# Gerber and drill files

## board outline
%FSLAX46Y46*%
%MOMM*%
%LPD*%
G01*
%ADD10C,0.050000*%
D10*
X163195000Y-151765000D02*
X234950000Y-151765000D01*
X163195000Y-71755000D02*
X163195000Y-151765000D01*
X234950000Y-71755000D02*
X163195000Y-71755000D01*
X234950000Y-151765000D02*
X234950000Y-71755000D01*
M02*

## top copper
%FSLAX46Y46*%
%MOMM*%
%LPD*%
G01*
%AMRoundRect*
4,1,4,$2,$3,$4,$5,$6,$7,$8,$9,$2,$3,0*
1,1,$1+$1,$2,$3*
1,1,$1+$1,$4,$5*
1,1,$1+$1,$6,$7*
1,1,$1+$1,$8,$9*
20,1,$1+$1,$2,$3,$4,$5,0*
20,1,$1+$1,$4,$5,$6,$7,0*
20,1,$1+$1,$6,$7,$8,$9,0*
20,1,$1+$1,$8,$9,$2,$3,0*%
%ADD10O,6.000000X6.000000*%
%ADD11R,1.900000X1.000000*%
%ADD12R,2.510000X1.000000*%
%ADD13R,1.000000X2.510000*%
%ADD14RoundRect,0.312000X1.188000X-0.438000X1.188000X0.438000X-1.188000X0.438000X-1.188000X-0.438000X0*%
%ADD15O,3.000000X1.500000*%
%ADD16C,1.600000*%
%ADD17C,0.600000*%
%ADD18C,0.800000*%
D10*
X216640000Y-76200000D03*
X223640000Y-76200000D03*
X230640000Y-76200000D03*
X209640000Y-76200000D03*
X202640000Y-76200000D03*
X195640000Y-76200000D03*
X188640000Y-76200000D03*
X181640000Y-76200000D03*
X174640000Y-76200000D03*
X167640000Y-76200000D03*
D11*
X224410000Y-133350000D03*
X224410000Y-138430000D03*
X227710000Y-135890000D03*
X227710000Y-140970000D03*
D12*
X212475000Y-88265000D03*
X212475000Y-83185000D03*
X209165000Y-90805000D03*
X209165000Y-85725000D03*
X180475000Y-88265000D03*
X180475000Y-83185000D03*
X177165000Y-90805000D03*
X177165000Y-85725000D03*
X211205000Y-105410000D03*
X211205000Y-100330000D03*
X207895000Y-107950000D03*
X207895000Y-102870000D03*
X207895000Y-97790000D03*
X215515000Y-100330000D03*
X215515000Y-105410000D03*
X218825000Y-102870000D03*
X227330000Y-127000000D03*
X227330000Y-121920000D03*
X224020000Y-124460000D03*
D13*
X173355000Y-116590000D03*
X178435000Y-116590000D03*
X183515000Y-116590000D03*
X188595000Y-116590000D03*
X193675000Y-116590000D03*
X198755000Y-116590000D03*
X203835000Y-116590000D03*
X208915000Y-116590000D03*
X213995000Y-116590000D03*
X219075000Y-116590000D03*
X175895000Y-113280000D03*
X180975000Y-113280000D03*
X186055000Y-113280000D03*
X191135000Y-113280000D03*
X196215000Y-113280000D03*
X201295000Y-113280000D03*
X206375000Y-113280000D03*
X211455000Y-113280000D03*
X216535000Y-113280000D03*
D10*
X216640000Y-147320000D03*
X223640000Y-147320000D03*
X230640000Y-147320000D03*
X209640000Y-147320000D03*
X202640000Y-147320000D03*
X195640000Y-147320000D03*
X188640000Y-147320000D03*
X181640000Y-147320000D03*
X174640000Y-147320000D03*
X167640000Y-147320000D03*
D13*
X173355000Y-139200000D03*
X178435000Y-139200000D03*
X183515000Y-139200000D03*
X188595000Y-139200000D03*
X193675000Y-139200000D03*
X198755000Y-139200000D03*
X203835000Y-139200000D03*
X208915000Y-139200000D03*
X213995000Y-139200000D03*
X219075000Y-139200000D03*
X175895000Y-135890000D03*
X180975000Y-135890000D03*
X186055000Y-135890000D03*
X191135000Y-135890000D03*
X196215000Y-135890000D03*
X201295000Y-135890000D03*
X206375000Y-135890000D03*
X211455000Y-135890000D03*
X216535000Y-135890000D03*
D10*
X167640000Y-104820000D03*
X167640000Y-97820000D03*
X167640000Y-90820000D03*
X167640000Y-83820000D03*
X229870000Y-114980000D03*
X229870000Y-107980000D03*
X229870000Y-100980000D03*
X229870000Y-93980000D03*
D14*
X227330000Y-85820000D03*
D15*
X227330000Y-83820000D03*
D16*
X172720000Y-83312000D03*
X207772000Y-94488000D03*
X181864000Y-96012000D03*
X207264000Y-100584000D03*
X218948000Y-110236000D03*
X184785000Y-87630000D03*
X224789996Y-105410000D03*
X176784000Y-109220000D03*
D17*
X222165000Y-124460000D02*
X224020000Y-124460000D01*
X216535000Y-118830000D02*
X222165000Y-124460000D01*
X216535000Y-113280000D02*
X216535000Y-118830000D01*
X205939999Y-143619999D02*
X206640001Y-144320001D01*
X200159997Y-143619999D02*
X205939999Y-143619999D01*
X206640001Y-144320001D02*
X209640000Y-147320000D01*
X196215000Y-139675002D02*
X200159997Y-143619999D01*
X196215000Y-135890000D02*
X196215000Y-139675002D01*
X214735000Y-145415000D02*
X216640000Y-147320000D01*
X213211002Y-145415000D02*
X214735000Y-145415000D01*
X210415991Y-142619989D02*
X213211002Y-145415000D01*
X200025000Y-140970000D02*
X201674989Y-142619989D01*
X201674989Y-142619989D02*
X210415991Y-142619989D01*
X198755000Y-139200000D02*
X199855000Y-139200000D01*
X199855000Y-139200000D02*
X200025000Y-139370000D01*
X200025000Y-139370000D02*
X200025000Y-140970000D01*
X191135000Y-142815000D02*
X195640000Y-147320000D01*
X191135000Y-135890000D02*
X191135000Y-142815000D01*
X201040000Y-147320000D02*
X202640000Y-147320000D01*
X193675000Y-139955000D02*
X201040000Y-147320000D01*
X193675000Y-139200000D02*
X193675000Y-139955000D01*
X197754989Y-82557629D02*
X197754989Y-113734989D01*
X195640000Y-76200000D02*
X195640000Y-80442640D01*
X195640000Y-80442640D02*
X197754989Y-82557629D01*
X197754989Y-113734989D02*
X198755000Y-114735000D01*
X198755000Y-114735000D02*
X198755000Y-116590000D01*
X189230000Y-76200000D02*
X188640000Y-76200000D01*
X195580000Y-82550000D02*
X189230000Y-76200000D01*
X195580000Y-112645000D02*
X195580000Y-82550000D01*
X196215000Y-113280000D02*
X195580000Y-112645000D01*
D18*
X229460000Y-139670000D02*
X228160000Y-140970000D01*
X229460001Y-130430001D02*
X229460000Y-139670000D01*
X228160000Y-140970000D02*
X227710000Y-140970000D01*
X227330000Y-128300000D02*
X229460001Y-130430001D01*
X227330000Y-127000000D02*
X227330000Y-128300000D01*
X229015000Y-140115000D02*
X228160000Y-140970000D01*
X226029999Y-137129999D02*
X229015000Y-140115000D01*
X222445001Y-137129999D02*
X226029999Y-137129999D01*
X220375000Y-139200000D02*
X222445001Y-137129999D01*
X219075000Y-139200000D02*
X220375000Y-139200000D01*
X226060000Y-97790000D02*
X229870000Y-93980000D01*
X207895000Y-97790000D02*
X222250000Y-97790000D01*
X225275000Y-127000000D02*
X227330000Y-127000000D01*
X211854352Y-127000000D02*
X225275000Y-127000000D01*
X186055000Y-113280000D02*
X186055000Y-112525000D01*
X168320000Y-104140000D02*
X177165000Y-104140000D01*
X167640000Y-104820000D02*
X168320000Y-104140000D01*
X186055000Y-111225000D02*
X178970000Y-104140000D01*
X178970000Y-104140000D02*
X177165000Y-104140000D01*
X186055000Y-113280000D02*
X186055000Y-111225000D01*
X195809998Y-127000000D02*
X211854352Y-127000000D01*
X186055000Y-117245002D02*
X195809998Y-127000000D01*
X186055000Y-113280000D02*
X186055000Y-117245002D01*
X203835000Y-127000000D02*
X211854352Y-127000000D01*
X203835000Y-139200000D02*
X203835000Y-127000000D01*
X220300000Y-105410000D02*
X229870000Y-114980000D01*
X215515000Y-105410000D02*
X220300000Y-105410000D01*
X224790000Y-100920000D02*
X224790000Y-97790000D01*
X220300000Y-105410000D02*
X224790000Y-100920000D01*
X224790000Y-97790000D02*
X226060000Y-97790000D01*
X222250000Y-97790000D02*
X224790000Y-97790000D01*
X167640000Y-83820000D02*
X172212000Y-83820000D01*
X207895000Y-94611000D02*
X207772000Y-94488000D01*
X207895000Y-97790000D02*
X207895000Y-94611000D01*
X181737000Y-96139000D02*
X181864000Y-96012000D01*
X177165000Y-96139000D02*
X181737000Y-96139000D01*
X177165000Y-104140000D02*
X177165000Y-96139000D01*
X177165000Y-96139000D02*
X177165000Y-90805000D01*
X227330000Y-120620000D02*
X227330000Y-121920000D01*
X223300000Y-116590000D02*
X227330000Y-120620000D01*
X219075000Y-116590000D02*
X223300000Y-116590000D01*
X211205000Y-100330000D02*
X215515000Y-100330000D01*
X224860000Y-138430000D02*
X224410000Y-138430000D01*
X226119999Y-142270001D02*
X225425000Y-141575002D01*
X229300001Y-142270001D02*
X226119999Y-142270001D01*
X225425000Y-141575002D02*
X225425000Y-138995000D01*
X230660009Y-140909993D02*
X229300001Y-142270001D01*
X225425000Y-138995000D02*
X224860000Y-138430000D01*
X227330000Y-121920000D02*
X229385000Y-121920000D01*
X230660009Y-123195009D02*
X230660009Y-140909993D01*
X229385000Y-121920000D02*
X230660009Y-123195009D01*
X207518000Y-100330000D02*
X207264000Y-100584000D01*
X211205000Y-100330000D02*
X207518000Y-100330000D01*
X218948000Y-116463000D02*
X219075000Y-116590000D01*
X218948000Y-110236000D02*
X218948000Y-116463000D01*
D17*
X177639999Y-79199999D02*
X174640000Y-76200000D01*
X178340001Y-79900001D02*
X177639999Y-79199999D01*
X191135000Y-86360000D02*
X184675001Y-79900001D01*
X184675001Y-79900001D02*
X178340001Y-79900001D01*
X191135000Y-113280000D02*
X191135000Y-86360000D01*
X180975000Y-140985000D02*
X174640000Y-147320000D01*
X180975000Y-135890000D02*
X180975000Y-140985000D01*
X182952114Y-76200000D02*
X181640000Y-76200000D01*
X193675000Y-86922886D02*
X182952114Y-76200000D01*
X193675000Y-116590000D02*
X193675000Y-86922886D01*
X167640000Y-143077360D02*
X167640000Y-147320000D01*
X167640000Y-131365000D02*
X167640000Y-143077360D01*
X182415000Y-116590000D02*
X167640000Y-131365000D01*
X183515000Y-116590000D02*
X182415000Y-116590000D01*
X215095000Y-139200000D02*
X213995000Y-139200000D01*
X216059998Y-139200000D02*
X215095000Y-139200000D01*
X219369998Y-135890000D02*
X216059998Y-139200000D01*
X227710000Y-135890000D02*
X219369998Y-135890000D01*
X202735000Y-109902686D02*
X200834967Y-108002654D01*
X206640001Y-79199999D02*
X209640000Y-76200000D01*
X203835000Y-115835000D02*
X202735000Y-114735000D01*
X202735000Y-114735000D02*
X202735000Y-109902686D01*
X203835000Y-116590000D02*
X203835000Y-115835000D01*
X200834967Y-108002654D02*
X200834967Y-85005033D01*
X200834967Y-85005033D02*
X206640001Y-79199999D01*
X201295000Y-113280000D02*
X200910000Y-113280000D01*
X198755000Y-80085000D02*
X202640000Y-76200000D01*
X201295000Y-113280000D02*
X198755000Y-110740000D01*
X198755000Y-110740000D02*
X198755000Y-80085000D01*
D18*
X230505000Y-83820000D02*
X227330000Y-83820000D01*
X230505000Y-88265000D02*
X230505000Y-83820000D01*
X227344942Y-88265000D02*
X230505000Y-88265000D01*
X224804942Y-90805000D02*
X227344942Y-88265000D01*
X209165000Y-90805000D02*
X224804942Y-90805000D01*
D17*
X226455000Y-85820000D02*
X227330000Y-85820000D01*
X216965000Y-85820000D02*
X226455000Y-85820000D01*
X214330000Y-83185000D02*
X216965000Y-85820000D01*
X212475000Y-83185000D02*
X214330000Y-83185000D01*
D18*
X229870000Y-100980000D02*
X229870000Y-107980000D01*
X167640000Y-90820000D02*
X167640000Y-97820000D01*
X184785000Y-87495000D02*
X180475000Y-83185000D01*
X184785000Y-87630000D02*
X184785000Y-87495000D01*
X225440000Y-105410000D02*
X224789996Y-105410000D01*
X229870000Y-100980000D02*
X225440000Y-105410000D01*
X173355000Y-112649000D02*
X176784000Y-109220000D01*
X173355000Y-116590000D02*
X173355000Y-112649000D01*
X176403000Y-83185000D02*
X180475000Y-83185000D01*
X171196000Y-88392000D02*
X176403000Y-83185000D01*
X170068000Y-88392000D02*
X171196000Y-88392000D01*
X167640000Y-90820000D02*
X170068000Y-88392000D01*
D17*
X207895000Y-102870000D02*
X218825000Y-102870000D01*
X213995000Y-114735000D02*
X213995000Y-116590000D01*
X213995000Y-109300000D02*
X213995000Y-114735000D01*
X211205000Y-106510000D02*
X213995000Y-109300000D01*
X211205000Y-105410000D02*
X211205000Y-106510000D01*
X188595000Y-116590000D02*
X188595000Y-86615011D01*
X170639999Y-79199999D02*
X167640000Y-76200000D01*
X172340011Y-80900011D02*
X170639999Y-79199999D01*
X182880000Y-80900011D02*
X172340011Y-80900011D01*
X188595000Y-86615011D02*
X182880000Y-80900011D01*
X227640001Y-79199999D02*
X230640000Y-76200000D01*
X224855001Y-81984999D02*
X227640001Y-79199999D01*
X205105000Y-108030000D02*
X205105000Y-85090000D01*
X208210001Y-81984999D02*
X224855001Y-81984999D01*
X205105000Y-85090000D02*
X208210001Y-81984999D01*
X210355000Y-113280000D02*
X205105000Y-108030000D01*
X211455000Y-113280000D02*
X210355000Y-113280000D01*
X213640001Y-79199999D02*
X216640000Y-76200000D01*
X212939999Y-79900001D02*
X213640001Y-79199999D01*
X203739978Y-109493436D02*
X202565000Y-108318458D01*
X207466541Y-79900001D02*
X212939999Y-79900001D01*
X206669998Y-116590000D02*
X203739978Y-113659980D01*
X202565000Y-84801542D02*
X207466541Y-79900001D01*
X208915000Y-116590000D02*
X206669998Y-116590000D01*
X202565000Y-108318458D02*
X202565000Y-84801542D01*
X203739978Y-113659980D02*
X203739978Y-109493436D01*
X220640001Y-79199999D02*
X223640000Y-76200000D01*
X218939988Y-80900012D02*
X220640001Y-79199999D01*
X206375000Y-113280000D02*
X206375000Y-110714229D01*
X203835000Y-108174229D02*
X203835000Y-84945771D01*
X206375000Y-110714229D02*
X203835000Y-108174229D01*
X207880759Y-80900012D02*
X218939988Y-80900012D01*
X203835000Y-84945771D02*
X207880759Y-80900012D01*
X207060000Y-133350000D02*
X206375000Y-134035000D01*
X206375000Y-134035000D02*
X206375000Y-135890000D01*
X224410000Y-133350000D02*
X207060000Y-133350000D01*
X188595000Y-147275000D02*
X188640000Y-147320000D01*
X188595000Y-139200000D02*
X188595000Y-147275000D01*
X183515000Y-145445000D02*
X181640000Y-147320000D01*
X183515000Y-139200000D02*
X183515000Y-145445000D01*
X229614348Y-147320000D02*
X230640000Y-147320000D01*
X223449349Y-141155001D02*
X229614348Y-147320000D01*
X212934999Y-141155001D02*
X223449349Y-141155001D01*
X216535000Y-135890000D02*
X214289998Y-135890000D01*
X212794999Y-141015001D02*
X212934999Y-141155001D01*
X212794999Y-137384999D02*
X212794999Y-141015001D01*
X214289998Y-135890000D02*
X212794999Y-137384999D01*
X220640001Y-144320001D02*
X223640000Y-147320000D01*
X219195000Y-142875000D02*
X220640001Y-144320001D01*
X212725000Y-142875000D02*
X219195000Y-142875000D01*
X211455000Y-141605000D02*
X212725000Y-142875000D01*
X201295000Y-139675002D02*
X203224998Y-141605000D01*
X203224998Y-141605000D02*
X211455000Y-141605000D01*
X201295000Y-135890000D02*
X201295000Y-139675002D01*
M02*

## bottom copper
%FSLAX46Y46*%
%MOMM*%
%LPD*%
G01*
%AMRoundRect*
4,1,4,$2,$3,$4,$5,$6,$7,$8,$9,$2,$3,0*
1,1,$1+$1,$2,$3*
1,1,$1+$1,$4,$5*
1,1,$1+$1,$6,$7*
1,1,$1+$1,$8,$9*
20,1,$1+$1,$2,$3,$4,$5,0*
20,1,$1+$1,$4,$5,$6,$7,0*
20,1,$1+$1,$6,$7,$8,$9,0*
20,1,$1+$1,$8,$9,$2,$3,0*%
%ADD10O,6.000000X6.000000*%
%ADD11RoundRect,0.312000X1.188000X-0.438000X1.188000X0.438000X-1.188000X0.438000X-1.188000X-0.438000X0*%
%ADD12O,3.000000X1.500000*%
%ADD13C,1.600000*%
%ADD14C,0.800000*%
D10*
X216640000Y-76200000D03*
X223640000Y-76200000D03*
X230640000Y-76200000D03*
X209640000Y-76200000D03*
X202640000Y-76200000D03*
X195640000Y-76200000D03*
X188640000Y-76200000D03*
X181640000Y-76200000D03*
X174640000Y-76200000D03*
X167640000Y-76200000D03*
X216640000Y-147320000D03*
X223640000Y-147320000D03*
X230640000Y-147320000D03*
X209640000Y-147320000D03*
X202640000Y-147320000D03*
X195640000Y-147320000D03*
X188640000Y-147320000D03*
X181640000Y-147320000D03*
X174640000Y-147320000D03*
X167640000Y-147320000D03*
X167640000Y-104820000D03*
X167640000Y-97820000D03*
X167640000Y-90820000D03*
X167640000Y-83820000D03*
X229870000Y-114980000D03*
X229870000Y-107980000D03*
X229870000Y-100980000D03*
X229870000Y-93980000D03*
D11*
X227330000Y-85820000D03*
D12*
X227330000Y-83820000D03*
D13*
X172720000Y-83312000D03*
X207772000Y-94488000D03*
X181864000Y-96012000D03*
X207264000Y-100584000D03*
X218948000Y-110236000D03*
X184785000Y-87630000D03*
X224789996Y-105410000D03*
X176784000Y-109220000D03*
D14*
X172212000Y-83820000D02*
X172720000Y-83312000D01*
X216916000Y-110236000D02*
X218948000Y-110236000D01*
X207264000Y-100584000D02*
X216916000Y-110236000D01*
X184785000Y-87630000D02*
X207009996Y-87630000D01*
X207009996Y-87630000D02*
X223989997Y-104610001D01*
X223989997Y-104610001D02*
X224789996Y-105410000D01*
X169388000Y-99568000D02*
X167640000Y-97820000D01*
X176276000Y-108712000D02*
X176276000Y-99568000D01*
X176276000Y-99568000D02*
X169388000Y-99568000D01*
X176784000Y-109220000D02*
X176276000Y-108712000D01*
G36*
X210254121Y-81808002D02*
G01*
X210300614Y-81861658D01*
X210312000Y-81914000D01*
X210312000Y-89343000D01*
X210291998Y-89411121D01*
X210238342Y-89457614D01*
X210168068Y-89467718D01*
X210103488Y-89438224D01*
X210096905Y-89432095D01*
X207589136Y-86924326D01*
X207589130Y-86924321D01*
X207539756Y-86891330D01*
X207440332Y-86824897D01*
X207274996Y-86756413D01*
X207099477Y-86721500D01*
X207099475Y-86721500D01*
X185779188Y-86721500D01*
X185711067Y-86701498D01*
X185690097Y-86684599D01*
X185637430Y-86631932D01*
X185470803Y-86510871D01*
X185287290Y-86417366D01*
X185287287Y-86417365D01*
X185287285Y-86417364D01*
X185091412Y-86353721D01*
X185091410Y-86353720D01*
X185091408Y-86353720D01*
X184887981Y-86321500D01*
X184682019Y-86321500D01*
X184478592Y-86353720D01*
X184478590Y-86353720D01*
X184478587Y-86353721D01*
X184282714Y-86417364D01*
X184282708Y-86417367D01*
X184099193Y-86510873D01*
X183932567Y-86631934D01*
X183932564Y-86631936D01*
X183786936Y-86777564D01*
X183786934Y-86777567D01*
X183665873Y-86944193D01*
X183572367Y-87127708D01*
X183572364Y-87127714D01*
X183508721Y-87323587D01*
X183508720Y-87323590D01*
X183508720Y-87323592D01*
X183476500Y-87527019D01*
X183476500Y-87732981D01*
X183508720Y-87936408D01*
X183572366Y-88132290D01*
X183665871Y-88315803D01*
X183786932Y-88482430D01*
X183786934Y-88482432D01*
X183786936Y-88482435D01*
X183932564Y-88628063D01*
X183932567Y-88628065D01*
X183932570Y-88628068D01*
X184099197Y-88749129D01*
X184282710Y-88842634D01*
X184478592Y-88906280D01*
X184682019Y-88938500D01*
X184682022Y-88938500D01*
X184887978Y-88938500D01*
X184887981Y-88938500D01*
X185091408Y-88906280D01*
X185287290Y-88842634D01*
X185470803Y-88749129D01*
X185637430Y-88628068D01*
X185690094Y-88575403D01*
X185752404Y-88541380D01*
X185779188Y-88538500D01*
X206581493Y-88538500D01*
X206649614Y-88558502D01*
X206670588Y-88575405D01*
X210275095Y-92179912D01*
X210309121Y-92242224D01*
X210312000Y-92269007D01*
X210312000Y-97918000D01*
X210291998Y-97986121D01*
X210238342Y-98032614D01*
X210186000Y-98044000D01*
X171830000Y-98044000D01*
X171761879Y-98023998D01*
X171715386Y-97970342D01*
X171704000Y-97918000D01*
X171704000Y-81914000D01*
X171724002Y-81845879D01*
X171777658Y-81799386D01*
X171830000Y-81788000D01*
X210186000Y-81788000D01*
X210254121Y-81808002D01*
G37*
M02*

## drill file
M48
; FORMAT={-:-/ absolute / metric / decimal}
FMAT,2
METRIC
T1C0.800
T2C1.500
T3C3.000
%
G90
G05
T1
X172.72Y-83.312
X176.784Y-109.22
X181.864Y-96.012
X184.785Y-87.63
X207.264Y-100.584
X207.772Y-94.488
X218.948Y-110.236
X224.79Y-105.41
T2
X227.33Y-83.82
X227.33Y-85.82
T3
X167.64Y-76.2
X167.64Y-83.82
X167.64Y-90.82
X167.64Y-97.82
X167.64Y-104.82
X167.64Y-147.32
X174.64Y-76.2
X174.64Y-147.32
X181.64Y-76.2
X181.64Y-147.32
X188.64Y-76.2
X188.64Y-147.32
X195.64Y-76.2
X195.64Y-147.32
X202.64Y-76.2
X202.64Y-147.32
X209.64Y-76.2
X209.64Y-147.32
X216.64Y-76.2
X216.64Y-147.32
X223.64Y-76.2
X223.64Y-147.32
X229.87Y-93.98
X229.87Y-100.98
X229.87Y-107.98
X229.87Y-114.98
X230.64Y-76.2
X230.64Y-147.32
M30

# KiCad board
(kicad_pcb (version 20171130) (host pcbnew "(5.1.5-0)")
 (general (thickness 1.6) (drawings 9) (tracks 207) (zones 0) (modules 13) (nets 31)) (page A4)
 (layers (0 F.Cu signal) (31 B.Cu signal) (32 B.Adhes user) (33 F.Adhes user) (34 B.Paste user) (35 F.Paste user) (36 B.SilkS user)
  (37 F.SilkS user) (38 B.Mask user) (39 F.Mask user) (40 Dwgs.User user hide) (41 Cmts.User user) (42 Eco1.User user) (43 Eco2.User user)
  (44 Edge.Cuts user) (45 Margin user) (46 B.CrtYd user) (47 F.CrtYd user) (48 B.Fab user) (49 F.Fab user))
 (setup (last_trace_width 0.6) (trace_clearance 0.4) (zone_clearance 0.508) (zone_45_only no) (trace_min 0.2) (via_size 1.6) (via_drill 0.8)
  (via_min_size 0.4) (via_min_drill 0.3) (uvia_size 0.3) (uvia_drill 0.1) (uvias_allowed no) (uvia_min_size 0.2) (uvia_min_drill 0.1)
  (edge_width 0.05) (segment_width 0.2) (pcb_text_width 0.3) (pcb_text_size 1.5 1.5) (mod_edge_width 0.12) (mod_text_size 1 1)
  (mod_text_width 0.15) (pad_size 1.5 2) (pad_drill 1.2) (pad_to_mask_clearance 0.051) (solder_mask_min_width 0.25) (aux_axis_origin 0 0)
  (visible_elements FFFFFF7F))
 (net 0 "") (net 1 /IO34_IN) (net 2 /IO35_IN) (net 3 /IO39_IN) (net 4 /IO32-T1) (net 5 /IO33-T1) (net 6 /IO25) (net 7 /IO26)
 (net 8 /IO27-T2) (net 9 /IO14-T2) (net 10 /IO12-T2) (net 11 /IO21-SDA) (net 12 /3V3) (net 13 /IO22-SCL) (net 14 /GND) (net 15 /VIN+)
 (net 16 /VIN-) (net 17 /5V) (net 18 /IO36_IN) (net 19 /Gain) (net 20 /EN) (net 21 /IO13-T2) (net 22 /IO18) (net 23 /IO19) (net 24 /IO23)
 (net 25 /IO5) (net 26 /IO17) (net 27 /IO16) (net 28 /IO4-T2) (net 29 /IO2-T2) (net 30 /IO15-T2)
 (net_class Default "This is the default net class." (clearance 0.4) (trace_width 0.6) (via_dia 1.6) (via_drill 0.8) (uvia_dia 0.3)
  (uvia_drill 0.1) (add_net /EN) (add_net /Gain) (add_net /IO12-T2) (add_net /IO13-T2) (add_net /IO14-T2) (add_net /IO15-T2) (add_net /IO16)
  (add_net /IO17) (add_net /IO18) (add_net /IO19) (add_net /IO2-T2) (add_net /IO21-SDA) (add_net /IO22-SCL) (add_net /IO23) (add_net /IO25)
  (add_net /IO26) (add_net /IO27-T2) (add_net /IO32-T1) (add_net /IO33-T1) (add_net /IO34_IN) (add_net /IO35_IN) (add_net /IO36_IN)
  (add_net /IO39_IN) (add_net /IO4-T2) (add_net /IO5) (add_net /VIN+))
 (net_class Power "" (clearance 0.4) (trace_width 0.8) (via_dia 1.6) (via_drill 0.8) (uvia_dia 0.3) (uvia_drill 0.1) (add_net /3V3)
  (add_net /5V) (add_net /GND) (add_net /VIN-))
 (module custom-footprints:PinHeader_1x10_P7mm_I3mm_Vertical (layer F.Cu) (at 167.64 76.2 90)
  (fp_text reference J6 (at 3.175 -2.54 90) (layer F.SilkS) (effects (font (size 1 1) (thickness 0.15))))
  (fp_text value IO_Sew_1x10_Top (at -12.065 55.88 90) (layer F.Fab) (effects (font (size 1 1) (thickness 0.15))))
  (pad 8 thru_hole oval (at 0 49 90) (size 6 6) (drill 3) (layers *.Cu *.Mask) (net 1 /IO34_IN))
  (pad 9 thru_hole oval (at 0 56 90) (size 6 6) (drill 3) (layers *.Cu *.Mask) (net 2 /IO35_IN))
  (pad 10 thru_hole oval (at 0 63 90) (size 6 6) (drill 3) (layers *.Cu *.Mask) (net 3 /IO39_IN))
  (pad 7 thru_hole oval (at 0 42 90) (size 6 6) (drill 3) (layers *.Cu *.Mask) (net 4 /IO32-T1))
  (pad 6 thru_hole oval (at 0 35 90) (size 6 6) (drill 3) (layers *.Cu *.Mask) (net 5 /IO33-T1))
  (pad 5 thru_hole oval (at 0 28 90) (size 6 6) (drill 3) (layers *.Cu *.Mask) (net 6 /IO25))
  (pad 4 thru_hole oval (at 0 21 90) (size 6 6) (drill 3) (layers *.Cu *.Mask) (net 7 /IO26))
  (pad 3 thru_hole oval (at 0 14 90) (size 6 6) (drill 3) (layers *.Cu *.Mask) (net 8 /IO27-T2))
  (pad 2 thru_hole oval (at 0 7 90) (size 6 6) (drill 3) (layers *.Cu *.Mask) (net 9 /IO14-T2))
  (pad 1 thru_hole oval (at 0 0 90) (size 6 6) (drill 3) (layers *.Cu *.Mask) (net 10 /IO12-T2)))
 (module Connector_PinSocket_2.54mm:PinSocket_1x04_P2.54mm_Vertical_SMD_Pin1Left (layer F.Cu) (at 226.06 137.16 180)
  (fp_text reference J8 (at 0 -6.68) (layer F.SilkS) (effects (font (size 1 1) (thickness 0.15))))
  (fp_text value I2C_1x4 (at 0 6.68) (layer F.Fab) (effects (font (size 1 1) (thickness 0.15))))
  (pad 4 smd rect (at 1.65 3.81 180) (size 1.9 1) (layers F.Cu F.Paste F.Mask) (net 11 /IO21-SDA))
  (pad 2 smd rect (at 1.65 -1.27 180) (size 1.9 1) (layers F.Cu F.Paste F.Mask) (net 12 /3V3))
  (pad 3 smd rect (at -1.65 1.27 180) (size 1.9 1) (layers F.Cu F.Paste F.Mask) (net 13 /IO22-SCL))
  (pad 1 smd rect (at -1.65 -3.81 180) (size 1.9 1) (layers F.Cu F.Paste F.Mask) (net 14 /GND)))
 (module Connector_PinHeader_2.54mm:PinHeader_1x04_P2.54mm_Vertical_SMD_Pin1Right (layer F.Cu) (at 210.82 86.995)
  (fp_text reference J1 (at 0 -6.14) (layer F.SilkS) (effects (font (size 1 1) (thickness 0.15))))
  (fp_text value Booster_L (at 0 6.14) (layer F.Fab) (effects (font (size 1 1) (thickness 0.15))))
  (pad 3 smd rect (at 1.655 1.27) (size 2.51 1) (layers F.Cu F.Paste F.Mask))
  (pad 1 smd rect (at 1.655 -3.81) (size 2.51 1) (layers F.Cu F.Paste F.Mask) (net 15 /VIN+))
  (pad 4 smd rect (at -1.655 3.81) (size 2.51 1) (layers F.Cu F.Paste F.Mask) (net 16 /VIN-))
  (pad 2 smd rect (at -1.655 -1.27) (size 2.51 1) (layers F.Cu F.Paste F.Mask)))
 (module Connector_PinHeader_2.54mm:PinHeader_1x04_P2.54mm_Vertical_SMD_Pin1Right (layer F.Cu) (at 178.82 86.995)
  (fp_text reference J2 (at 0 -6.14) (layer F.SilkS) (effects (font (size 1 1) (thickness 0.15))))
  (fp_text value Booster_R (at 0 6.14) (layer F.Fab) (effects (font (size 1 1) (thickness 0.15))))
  (pad 3 smd rect (at 1.655 1.27) (size 2.51 1) (layers F.Cu F.Paste F.Mask))
  (pad 1 smd rect (at 1.655 -3.81) (size 2.51 1) (layers F.Cu F.Paste F.Mask) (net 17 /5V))
  (pad 4 smd rect (at -1.655 3.81) (size 2.51 1) (layers F.Cu F.Paste F.Mask) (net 14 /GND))
  (pad 2 smd rect (at -1.655 -1.27) (size 2.51 1) (layers F.Cu F.Paste F.Mask)))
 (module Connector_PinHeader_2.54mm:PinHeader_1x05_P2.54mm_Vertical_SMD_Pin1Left (layer F.Cu) (at 209.55 102.87)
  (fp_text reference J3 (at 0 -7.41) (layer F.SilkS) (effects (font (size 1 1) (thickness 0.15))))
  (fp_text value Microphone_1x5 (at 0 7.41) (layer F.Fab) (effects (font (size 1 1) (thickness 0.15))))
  (pad 4 smd rect (at 1.655 2.54) (size 2.51 1) (layers F.Cu F.Paste F.Mask) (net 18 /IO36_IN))
  (pad 2 smd rect (at 1.655 -2.54) (size 2.51 1) (layers F.Cu F.Paste F.Mask) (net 12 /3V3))
  (pad 5 smd rect (at -1.655 5.08) (size 2.51 1) (layers F.Cu F.Paste F.Mask))
  (pad 3 smd rect (at -1.655 0) (size 2.51 1) (layers F.Cu F.Paste F.Mask) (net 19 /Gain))
  (pad 1 smd rect (at -1.655 -5.08) (size 2.51 1) (layers F.Cu F.Paste F.Mask) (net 14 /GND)))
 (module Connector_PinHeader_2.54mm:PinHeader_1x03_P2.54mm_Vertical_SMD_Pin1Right (layer F.Cu) (at 217.17 102.87 180)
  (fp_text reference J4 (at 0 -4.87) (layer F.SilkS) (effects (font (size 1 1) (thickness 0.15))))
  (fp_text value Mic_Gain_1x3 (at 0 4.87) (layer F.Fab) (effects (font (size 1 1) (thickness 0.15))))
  (pad 3 smd rect (at 1.655 2.54 180) (size 2.51 1) (layers F.Cu F.Paste F.Mask) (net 12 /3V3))
  (pad 1 smd rect (at 1.655 -2.54 180) (size 2.51 1) (layers F.Cu F.Paste F.Mask) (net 14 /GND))
  (pad 2 smd rect (at -1.655 0 180) (size 2.51 1) (layers F.Cu F.Paste F.Mask) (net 19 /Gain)))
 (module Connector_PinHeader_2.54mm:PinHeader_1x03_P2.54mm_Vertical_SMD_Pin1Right (layer F.Cu) (at 225.675 124.46)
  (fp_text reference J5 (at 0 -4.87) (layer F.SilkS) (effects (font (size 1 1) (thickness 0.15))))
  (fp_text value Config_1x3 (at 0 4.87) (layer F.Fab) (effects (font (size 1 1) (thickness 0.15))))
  (pad 3 smd rect (at 1.655 2.54) (size 2.51 1) (layers F.Cu F.Paste F.Mask) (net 14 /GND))
  (pad 1 smd rect (at 1.655 -2.54) (size 2.51 1) (layers F.Cu F.Paste F.Mask) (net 12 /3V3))
  (pad 2 smd rect (at -1.655 0) (size 2.51 1) (layers F.Cu F.Paste F.Mask) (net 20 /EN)))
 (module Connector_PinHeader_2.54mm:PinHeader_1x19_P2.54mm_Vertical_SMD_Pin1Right (layer F.Cu) (at 196.215 114.935 270)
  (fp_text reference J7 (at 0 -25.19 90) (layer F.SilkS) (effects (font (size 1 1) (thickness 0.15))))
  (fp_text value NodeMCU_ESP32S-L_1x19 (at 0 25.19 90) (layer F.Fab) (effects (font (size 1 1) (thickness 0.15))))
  (pad 19 smd rect (at 1.655 22.86 270) (size 2.51 1) (layers F.Cu F.Paste F.Mask) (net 17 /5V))
  (pad 17 smd rect (at 1.655 17.78 270) (size 2.51 1) (layers F.Cu F.Paste F.Mask))
  (pad 15 smd rect (at 1.655 12.7 270) (size 2.51 1) (layers F.Cu F.Paste F.Mask) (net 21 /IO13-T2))
  (pad 13 smd rect (at 1.655 7.62 270) (size 2.51 1) (layers F.Cu F.Paste F.Mask) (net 10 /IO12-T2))
  (pad 11 smd rect (at 1.655 2.54 270) (size 2.51 1) (layers F.Cu F.Paste F.Mask) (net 8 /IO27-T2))
  (pad 9 smd rect (at 1.655 -2.54 270) (size 2.51 1) (layers F.Cu F.Paste F.Mask) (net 6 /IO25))
  (pad 7 smd rect (at 1.655 -7.62 270) (size 2.51 1) (layers F.Cu F.Paste F.Mask) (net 4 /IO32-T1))
  (pad 5 smd rect (at 1.655 -12.7 270) (size 2.51 1) (layers F.Cu F.Paste F.Mask) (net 1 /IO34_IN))
  (pad 3 smd rect (at 1.655 -17.78 270) (size 2.51 1) (layers F.Cu F.Paste F.Mask) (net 18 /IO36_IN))
  (pad 1 smd rect (at 1.655 -22.86 270) (size 2.51 1) (layers F.Cu F.Paste F.Mask) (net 12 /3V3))
  (pad 18 smd rect (at -1.655 20.32 270) (size 2.51 1) (layers F.Cu F.Paste F.Mask))
  (pad 16 smd rect (at -1.655 15.24 270) (size 2.51 1) (layers F.Cu F.Paste F.Mask))
  (pad 14 smd rect (at -1.655 10.16 270) (size 2.51 1) (layers F.Cu F.Paste F.Mask) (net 14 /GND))
  (pad 12 smd rect (at -1.655 5.08 270) (size 2.51 1) (layers F.Cu F.Paste F.Mask) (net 9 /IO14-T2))
  (pad 10 smd rect (at -1.655 0 270) (size 2.51 1) (layers F.Cu F.Paste F.Mask) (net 7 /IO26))
  (pad 8 smd rect (at -1.655 -5.08 270) (size 2.51 1) (layers F.Cu F.Paste F.Mask) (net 5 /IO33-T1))
  (pad 6 smd rect (at -1.655 -10.16 270) (size 2.51 1) (layers F.Cu F.Paste F.Mask) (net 2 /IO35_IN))
  (pad 4 smd rect (at -1.655 -15.24 270) (size 2.51 1) (layers F.Cu F.Paste F.Mask) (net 3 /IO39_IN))
  (pad 2 smd rect (at -1.655 -20.32 270) (size 2.51 1) (layers F.Cu F.Paste F.Mask) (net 20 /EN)))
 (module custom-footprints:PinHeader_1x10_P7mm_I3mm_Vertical (layer F.Cu) (at 167.64 147.32 90)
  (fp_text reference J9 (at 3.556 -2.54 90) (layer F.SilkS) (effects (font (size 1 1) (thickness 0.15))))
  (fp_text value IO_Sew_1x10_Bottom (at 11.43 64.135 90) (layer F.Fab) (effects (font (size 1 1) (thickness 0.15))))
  (pad 8 thru_hole oval (at 0 49 90) (size 6 6) (drill 3) (layers *.Cu *.Mask) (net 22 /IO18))
  (pad 9 thru_hole oval (at 0 56 90) (size 6 6) (drill 3) (layers *.Cu *.Mask) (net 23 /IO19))
  (pad 10 thru_hole oval (at 0 63 90) (size 6 6) (drill 3) (layers *.Cu *.Mask) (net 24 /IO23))
  (pad 7 thru_hole oval (at 0 42 90) (size 6 6) (drill 3) (layers *.Cu *.Mask) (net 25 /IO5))
  (pad 6 thru_hole oval (at 0 35 90) (size 6 6) (drill 3) (layers *.Cu *.Mask) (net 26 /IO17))
  (pad 5 thru_hole oval (at 0 28 90) (size 6 6) (drill 3) (layers *.Cu *.Mask) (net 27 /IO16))
  (pad 4 thru_hole oval (at 0 21 90) (size 6 6) (drill 3) (layers *.Cu *.Mask) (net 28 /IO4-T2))
  (pad 3 thru_hole oval (at 0 14 90) (size 6 6) (drill 3) (layers *.Cu *.Mask) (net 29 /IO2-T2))
  (pad 2 thru_hole oval (at 0 7 90) (size 6 6) (drill 3) (layers *.Cu *.Mask) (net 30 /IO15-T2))
  (pad 1 thru_hole oval (at 0 0 90) (size 6 6) (drill 3) (layers *.Cu *.Mask) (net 21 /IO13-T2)))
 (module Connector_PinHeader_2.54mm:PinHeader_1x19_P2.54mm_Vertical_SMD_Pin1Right (layer F.Cu) (at 196.215 137.545 270)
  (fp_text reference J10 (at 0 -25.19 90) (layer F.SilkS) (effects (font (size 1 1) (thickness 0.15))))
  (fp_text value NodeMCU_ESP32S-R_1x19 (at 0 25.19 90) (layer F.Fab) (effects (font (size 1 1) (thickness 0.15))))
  (pad 19 smd rect (at 1.655 22.86 270) (size 2.51 1) (layers F.Cu F.Paste F.Mask))
  (pad 17 smd rect (at 1.655 17.78 270) (size 2.51 1) (layers F.Cu F.Paste F.Mask))
  (pad 15 smd rect (at 1.655 12.7 270) (size 2.51 1) (layers F.Cu F.Paste F.Mask) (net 29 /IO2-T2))
  (pad 13 smd rect (at 1.655 7.62 270) (size 2.51 1) (layers F.Cu F.Paste F.Mask) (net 28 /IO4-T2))
  (pad 11 smd rect (at 1.655 2.54 270) (size 2.51 1) (layers F.Cu F.Paste F.Mask) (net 26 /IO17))
  (pad 9 smd rect (at 1.655 -2.54 270) (size 2.51 1) (layers F.Cu F.Paste F.Mask) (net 22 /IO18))
  (pad 7 smd rect (at 1.655 -7.62 270) (size 2.51 1) (layers F.Cu F.Paste F.Mask) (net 14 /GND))
  (pad 5 smd rect (at 1.655 -12.7 270) (size 2.51 1) (layers F.Cu F.Paste F.Mask))
  (pad 3 smd rect (at 1.655 -17.78 270) (size 2.51 1) (layers F.Cu F.Paste F.Mask) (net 13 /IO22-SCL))
  (pad 1 smd rect (at 1.655 -22.86 270) (size 2.51 1) (layers F.Cu F.Paste F.Mask) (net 14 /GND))
  (pad 18 smd rect (at -1.655 20.32 270) (size 2.51 1) (layers F.Cu F.Paste F.Mask))
  (pad 16 smd rect (at -1.655 15.24 270) (size 2.51 1) (layers F.Cu F.Paste F.Mask) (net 30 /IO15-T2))
  (pad 14 smd rect (at -1.655 10.16 270) (size 2.51 1) (layers F.Cu F.Paste F.Mask))
  (pad 12 smd rect (at -1.655 5.08 270) (size 2.51 1) (layers F.Cu F.Paste F.Mask) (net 27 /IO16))
  (pad 10 smd rect (at -1.655 0 270) (size 2.51 1) (layers F.Cu F.Paste F.Mask) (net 25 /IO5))
  (pad 8 smd rect (at -1.655 -5.08 270) (size 2.51 1) (layers F.Cu F.Paste F.Mask) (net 23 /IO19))
  (pad 6 smd rect (at -1.655 -10.16 270) (size 2.51 1) (layers F.Cu F.Paste F.Mask) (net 11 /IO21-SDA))
  (pad 4 smd rect (at -1.655 -15.24 270) (size 2.51 1) (layers F.Cu F.Paste F.Mask))
  (pad 2 smd rect (at -1.655 -20.32 270) (size 2.51 1) (layers F.Cu F.Paste F.Mask) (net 24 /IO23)))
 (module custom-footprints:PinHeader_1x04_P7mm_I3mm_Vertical (layer F.Cu) (at 167.64 83.82)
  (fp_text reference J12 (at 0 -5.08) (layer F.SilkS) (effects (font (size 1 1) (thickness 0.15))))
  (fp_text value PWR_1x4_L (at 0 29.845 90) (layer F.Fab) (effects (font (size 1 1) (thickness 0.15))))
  (pad 4 thru_hole oval (at 0 21) (size 6 6) (drill 3) (layers *.Cu *.Mask) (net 14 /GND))
  (pad 3 thru_hole oval (at 0 14) (size 6 6) (drill 3) (layers *.Cu *.Mask) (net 17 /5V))
  (pad 2 thru_hole oval (at 0 7) (size 6 6) (drill 3) (layers *.Cu *.Mask) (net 17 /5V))
  (pad 1 thru_hole oval (at 0 0) (size 6 6) (drill 3) (layers *.Cu *.Mask) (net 14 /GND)))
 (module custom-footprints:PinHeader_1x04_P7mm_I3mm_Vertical (layer F.Cu) (at 229.87 93.98)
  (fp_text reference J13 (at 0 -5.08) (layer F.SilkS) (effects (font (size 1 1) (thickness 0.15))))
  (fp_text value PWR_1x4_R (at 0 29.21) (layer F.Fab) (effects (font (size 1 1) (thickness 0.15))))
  (pad 4 thru_hole oval (at 0 21) (size 6 6) (drill 3) (layers *.Cu *.Mask) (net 14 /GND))
  (pad 3 thru_hole oval (at 0 14) (size 6 6) (drill 3) (layers *.Cu *.Mask) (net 17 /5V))
  (pad 2 thru_hole oval (at 0 7) (size 6 6) (drill 3) (layers *.Cu *.Mask) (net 17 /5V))
  (pad 1 thru_hole oval (at 0 0) (size 6 6) (drill 3) (layers *.Cu *.Mask) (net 14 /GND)))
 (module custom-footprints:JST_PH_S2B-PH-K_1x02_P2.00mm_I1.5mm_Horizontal (layer F.Cu) (at 227.33 85.82 90)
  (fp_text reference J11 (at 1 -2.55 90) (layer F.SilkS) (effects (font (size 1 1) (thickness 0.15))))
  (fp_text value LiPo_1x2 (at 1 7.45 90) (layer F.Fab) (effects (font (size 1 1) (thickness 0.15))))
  (pad 1 thru_hole roundrect (at 0 0 90) (size 1.5 3) (drill 1.5) (layers *.Cu *.Mask) (roundrect_rratio 0.208) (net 15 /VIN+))
  (pad 2 thru_hole oval (at 2 0 90) (size 1.5 3) (drill 1.5) (layers *.Cu *.Mask) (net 16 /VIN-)))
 (gr_line (start 163.195 151.765) (end 234.95 151.765) (layer Edge.Cuts) (width 0.05))
 (gr_line (start 163.195 71.755) (end 163.195 151.765) (layer Edge.Cuts) (width 0.05))
 (gr_line (start 234.95 71.755) (end 163.195 71.755) (layer Edge.Cuts) (width 0.05))
 (gr_line (start 234.95 151.765) (end 234.95 71.755) (layer Edge.Cuts) (width 0.05))
 (segment (start 222.165 124.46) (end 224.02 124.46) (width 0.6) (layer F.Cu) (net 20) (status 20))
 (segment (start 216.535 118.83) (end 222.165 124.46) (width 0.6) (layer F.Cu) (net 20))
 (segment (start 216.535 113.28) (end 216.535 118.83) (width 0.6) (layer F.Cu) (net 20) (status 10))
 (segment (start 205.939999 143.619999) (end 206.640001 144.320001) (width 0.6) (layer F.Cu) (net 25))
 (segment (start 200.159997 143.619999) (end 205.939999 143.619999) (width 0.6) (layer F.Cu) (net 25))
 (segment (start 206.640001 144.320001) (end 209.64 147.32) (width 0.6) (layer F.Cu) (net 25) (status 20))
 (segment (start 196.215 139.675002) (end 200.159997 143.619999) (width 0.6) (layer F.Cu) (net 25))
 (segment (start 196.215 135.89) (end 196.215 139.675002) (width 0.6) (layer F.Cu) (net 25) (status 10))
 (segment (start 214.735 145.415) (end 216.64 147.32) (width 0.6) (layer F.Cu) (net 22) (status 30))
 (segment (start 213.211002 145.415) (end 214.735 145.415) (width 0.6) (layer F.Cu) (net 22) (status 20))
 (segment (start 210.415991 142.619989) (end 213.211002 145.415) (width 0.6) (layer F.Cu) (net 22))
 (segment (start 200.025 140.97) (end 201.674989 142.619989) (width 0.6) (layer F.Cu) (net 22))
 (segment (start 201.674989 142.619989) (end 210.415991 142.619989) (width 0.6) (layer F.Cu) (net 22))
 (segment (start 198.755 139.2) (end 199.855 139.2) (width 0.6) (layer F.Cu) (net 22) (status 10))
 (segment (start 199.855 139.2) (end 200.025 139.37) (width 0.6) (layer F.Cu) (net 22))
 (segment (start 200.025 139.37) (end 200.025 140.97) (width 0.6) (layer F.Cu) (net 22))
 (segment (start 191.135 142.815) (end 195.64 147.32) (width 0.6) (layer F.Cu) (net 27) (status 20))
 (segment (start 191.135 135.89) (end 191.135 142.815) (width 0.6) (layer F.Cu) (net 27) (status 10))
 (segment (start 201.04 147.32) (end 202.64 147.32) (width 0.6) (layer F.Cu) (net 26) (status 30))
 (segment (start 193.675 139.955) (end 201.04 147.32) (width 0.6) (layer F.Cu) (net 26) (status 30))
 (segment (start 193.675 139.2) (end 193.675 139.955) (width 0.6) (layer F.Cu) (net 26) (status 30))
 (segment (start 197.754989 82.557629) (end 197.754989 113.734989) (width 0.6) (layer F.Cu) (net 6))
 (segment (start 195.64 76.2) (end 195.64 80.44264) (width 0.6) (layer F.Cu) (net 6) (status 10))
 (segment (start 195.64 80.44264) (end 197.754989 82.557629) (width 0.6) (layer F.Cu) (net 6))
 (segment (start 197.754989 113.734989) (end 198.755 114.735) (width 0.6) (layer F.Cu) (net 6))
 (segment (start 198.755 114.735) (end 198.755 116.59) (width 0.6) (layer F.Cu) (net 6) (status 20))
 (segment (start 189.23 76.2) (end 188.64 76.2) (width 0.6) (layer F.Cu) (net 7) (status 30))
 (segment (start 195.58 82.55) (end 189.23 76.2) (width 0.6) (layer F.Cu) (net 7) (status 20))
 (segment (start 195.58 112.645) (end 195.58 82.55) (width 0.6) (layer F.Cu) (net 7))
 (segment (start 196.215 113.28) (end 195.58 112.645) (width 0.6) (layer F.Cu) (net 7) (status 10))
 (segment (start 229.46 139.67) (end 228.16 140.97) (width 0.8) (layer F.Cu) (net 14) (status 20))
 (segment (start 229.460001 130.430001) (end 229.46 139.67) (width 0.8) (layer F.Cu) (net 14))
 (segment (start 228.16 140.97) (end 227.71 140.97) (width 0.8) (layer F.Cu) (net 14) (status 30))
 (segment (start 227.33 128.3) (end 229.460001 130.430001) (width 0.8) (layer F.Cu) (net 14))
 (segment (start 227.33 127) (end 227.33 128.3) (width 0.8) (layer F.Cu) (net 14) (status 10))
 (segment (start 229.015 140.115) (end 228.16 140.97) (width 0.8) (layer F.Cu) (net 14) (status 20))
 (segment (start 226.029999 137.129999) (end 229.015 140.115) (width 0.8) (layer F.Cu) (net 14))
 (segment (start 222.445001 137.129999) (end 226.029999 137.129999) (width 0.8) (layer F.Cu) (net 14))
 (segment (start 220.375 139.2) (end 222.445001 137.129999) (width 0.8) (layer F.Cu) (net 14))
 (segment (start 219.075 139.2) (end 220.375 139.2) (width 0.8) (layer F.Cu) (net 14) (status 10))
 (segment (start 226.06 97.79) (end 229.87 93.98) (width 0.8) (layer F.Cu) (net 14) (status 20))
 (segment (start 207.895 97.79) (end 222.25 97.79) (width 0.8) (layer F.Cu) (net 14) (status 10))
 (segment (start 225.275 127) (end 227.33 127) (width 0.8) (layer F.Cu) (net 14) (status 20))
 (segment (start 211.854352 127) (end 225.275 127) (width 0.8) (layer F.Cu) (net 14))
 (segment (start 186.055 113.28) (end 186.055 112.525) (width 0.8) (layer F.Cu) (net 14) (status 30))
 (segment (start 168.32 104.14) (end 177.165 104.14) (width 0.8) (layer F.Cu) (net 14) (status 10))
 (segment (start 167.64 104.82) (end 168.32 104.14) (width 0.8) (layer F.Cu) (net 14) (status 30))
 (segment (start 186.055 111.225) (end 178.97 104.14) (width 0.8) (layer F.Cu) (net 14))
 (segment (start 178.97 104.14) (end 177.165 104.14) (width 0.8) (layer F.Cu) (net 14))
 (segment (start 186.055 113.28) (end 186.055 111.225) (width 0.8) (layer F.Cu) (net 14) (status 10))
 (segment (start 195.809998 127) (end 211.854352 127) (width 0.8) (layer F.Cu) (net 14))
 (segment (start 186.055 117.245002) (end 195.809998 127) (width 0.8) (layer F.Cu) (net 14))
 (segment (start 186.055 113.28) (end 186.055 117.245002) (width 0.8) (layer F.Cu) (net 14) (status 10))
 (segment (start 203.835 127) (end 211.854352 127) (width 0.8) (layer F.Cu) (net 14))
 (segment (start 203.835 139.2) (end 203.835 127) (width 0.8) (layer F.Cu) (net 14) (status 10))
 (segment (start 220.3 105.41) (end 229.87 114.98) (width 0.8) (layer F.Cu) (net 14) (status 20))
 (segment (start 215.515 105.41) (end 220.3 105.41) (width 0.8) (layer F.Cu) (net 14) (status 10))
 (segment (start 224.79 100.92) (end 224.79 97.79) (width 0.8) (layer F.Cu) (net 14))
 (segment (start 220.3 105.41) (end 224.79 100.92) (width 0.8) (layer F.Cu) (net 14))
 (segment (start 224.79 97.79) (end 226.06 97.79) (width 0.8) (layer F.Cu) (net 14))
 (segment (start 222.25 97.79) (end 224.79 97.79) (width 0.8) (layer F.Cu) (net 14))
 (via (at 172.72 83.312) (size 1.6) (drill 0.8) (layers F.Cu B.Cu) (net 14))
 (segment (start 172.212 83.82) (end 172.72 83.312) (width 0.8) (layer B.Cu) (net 14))
 (segment (start 167.64 83.82) (end 172.212 83.82) (width 0.8) (layer F.Cu) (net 14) (status 10))
 (segment (start 207.895 94.611) (end 207.772 94.488) (width 0.8) (layer F.Cu) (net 14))
 (via (at 207.772 94.488) (size 1.6) (drill 0.8) (layers F.Cu B.Cu) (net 14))
 (segment (start 207.895 97.79) (end 207.895 94.611) (width 0.8) (layer F.Cu) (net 14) (status 10))
 (segment (start 181.737 96.139) (end 181.864 96.012) (width 0.8) (layer F.Cu) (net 14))
 (segment (start 177.165 96.139) (end 181.737 96.139) (width 0.8) (layer F.Cu) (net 14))
 (via (at 181.864 96.012) (size 1.6) (drill 0.8) (layers F.Cu B.Cu) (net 14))
 (segment (start 177.165 104.14) (end 177.165 96.139) (width 0.8) (layer F.Cu) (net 14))
 (segment (start 177.165 96.139) (end 177.165 90.805) (width 0.8) (layer F.Cu) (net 14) (status 20))
 (segment (start 227.33 120.62) (end 227.33 121.92) (width 0.8) (layer F.Cu) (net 12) (status 20))
 (segment (start 223.3 116.59) (end 227.33 120.62) (width 0.8) (layer F.Cu) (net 12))
 (segment (start 219.075 116.59) (end 223.3 116.59) (width 0.8) (layer F.Cu) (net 12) (status 10))
 (segment (start 211.205 100.33) (end 215.515 100.33) (width 0.8) (layer F.Cu) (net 12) (status 30))
 (segment (start 224.86 138.43) (end 224.41 138.43) (width 0.8) (layer F.Cu) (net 12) (status 30))
 (segment (start 226.119999 142.270001) (end 225.425 141.575002) (width 0.8) (layer F.Cu) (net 12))
 (segment (start 229.300001 142.270001) (end 226.119999 142.270001) (width 0.8) (layer F.Cu) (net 12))
 (segment (start 225.425 141.575002) (end 225.425 138.995) (width 0.8) (layer F.Cu) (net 12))
 (segment (start 230.660009 140.909993) (end 229.300001 142.270001) (width 0.8) (layer F.Cu) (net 12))
 (segment (start 225.425 138.995) (end 224.86 138.43) (width 0.8) (layer F.Cu) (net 12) (status 20))
 (segment (start 227.33 121.92) (end 229.385 121.92) (width 0.8) (layer F.Cu) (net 12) (status 10))
 (segment (start 230.660009 123.195009) (end 230.660009 140.909993) (width 0.8) (layer F.Cu) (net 12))
 (segment (start 229.385 121.92) (end 230.660009 123.195009) (width 0.8) (layer F.Cu) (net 12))
 (via (at 207.264 100.584) (size 1.6) (drill 0.8) (layers F.Cu B.Cu) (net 12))
 (segment (start 207.518 100.33) (end 207.264 100.584) (width 0.8) (layer F.Cu) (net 12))
 (segment (start 211.205 100.33) (end 207.518 100.33) (width 0.8) (layer F.Cu) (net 12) (status 10))
 (via (at 218.948 110.236) (size 1.6) (drill 0.8) (layers F.Cu B.Cu) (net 12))
 (segment (start 216.916 110.236) (end 218.948 110.236) (width 0.8) (layer B.Cu) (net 12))
 (segment (start 207.264 100.584) (end 216.916 110.236) (width 0.8) (layer B.Cu) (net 12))
 (segment (start 218.948 116.463) (end 219.075 116.59) (width 0.8) (layer F.Cu) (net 12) (status 30))
 (segment (start 218.948 110.236) (end 218.948 116.463) (width 0.8) (layer F.Cu) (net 12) (status 20))
 (segment (start 177.639999 79.199999) (end 174.64 76.2) (width 0.6) (layer F.Cu) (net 9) (status 20))
 (segment (start 178.340001 79.900001) (end 177.639999 79.199999) (width 0.6) (layer F.Cu) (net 9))
 (segment (start 191.135 86.36) (end 184.675001 79.900001) (width 0.6) (layer F.Cu) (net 9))
 (segment (start 184.675001 79.900001) (end 178.340001 79.900001) (width 0.6) (layer F.Cu) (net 9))
 (segment (start 191.135 113.28) (end 191.135 86.36) (width 0.6) (layer F.Cu) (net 9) (status 10))
 (segment (start 180.975 140.985) (end 174.64 147.32) (width 0.6) (layer F.Cu) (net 30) (status 20))
 (segment (start 180.975 135.89) (end 180.975 140.985) (width 0.6) (layer F.Cu) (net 30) (status 10))
 (segment (start 182.952114 76.2) (end 181.64 76.2) (width 0.6) (layer F.Cu) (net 8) (status 30))
 (segment (start 193.675 86.922886) (end 182.952114 76.2) (width 0.6) (layer F.Cu) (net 8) (status 20))
 (segment (start 193.675 116.59) (end 193.675 86.922886) (width 0.6) (layer F.Cu) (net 8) (status 10))
 (segment (start 167.64 143.07736) (end 167.64 147.32) (width 0.6) (layer F.Cu) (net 21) (status 20))
 (segment (start 167.64 131.365) (end 167.64 143.07736) (width 0.6) (layer F.Cu) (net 21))
 (segment (start 182.415 116.59) (end 167.64 131.365) (width 0.6) (layer F.Cu) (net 21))
 (segment (start 183.515 116.59) (end 182.415 116.59) (width 0.6) (layer F.Cu) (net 21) (status 10))
 (segment (start 215.095 139.2) (end 213.995 139.2) (width 0.6) (layer F.Cu) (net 13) (status 20))
 (segment (start 216.059998 139.2) (end 215.095 139.2) (width 0.6) (layer F.Cu) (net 13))
 (segment (start 219.369998 135.89) (end 216.059998 139.2) (width 0.6) (layer F.Cu) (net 13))
 (segment (start 227.71 135.89) (end 219.369998 135.89) (width 0.6) (layer F.Cu) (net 13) (status 10))
 (segment (start 202.735 109.902686) (end 200.834967 108.002654) (width 0.6) (layer F.Cu) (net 4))
 (segment (start 206.640001 79.199999) (end 209.64 76.2) (width 0.6) (layer F.Cu) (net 4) (status 20))
 (segment (start 203.835 115.835) (end 202.735 114.735) (width 0.6) (layer F.Cu) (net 4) (status 10))
 (segment (start 202.735 114.735) (end 202.735 109.902686) (width 0.6) (layer F.Cu) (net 4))
 (segment (start 203.835 116.59) (end 203.835 115.835) (width 0.6) (layer F.Cu) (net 4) (status 30))
 (segment (start 200.834967 108.002654) (end 200.834967 85.005033) (width 0.6) (layer F.Cu) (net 4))
 (segment (start 200.834967 85.005033) (end 206.640001 79.199999) (width 0.6) (layer F.Cu) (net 4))
 (segment (start 201.295 113.28) (end 200.91 113.28) (width 0.6) (layer F.Cu) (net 5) (status 30))
 (segment (start 198.755 80.085) (end 202.64 76.2) (width 0.6) (layer F.Cu) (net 5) (status 20))
 (segment (start 201.295 113.28) (end 198.755 110.74) (width 0.6) (layer F.Cu) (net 5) (status 10))
 (segment (start 198.755 110.74) (end 198.755 80.085) (width 0.6) (layer F.Cu) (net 5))
 (segment (start 230.505 83.82) (end 227.33 83.82) (width 0.8) (layer F.Cu) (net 16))
 (segment (start 230.505 88.265) (end 230.505 83.82) (width 0.8) (layer F.Cu) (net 16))
 (segment (start 227.344942 88.265) (end 230.505 88.265) (width 0.8) (layer F.Cu) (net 16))
 (segment (start 224.804942 90.805) (end 227.344942 88.265) (width 0.8) (layer F.Cu) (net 16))
 (segment (start 209.165 90.805) (end 224.804942 90.805) (width 0.8) (layer F.Cu) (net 16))
 (segment (start 226.455 85.82) (end 227.33 85.82) (width 0.6) (layer F.Cu) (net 15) (status 30))
 (segment (start 216.965 85.82) (end 226.455 85.82) (width 0.6) (layer F.Cu) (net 15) (status 20))
 (segment (start 214.33 83.185) (end 216.965 85.82) (width 0.6) (layer F.Cu) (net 15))
 (segment (start 212.475 83.185) (end 214.33 83.185) (width 0.6) (layer F.Cu) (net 15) (status 10))
 (segment (start 229.87 100.98) (end 229.87 107.98) (width 0.8) (layer F.Cu) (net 17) (status 30))
 (segment (start 167.64 90.82) (end 167.64 97.82) (width 0.8) (layer F.Cu) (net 17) (status 30))
 (via (at 184.785 87.63) (size 1.6) (drill 0.8) (layers F.Cu B.Cu) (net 17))
 (segment (start 184.785 87.495) (end 180.475 83.185) (width 0.8) (layer F.Cu) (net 17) (status 20))
 (segment (start 184.785 87.63) (end 184.785 87.495) (width 0.8) (layer F.Cu) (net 17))
 (segment (start 225.44 105.41) (end 224.789996 105.41) (width 0.8) (layer F.Cu) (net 17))
 (segment (start 229.87 100.98) (end 225.44 105.41) (width 0.8) (layer F.Cu) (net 17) (status 10))
 (segment (start 184.785 87.63) (end 207.009996 87.63) (width 0.8) (layer B.Cu) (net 17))
 (via (at 224.789996 105.41) (size 1.6) (drill 0.8) (layers F.Cu B.Cu) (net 17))
 (segment (start 207.009996 87.63) (end 223.989997 104.610001) (width 0.8) (layer B.Cu) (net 17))
 (segment (start 223.989997 104.610001) (end 224.789996 105.41) (width 0.8) (layer B.Cu) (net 17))
 (via (at 176.784 109.22) (size 1.6) (drill 0.8) (layers F.Cu B.Cu) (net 17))
 (segment (start 173.355 112.649) (end 176.784 109.22) (width 0.8) (layer F.Cu) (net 17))
 (segment (start 173.355 116.59) (end 173.355 112.649) (width 0.8) (layer F.Cu) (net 17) (status 10))
 (segment (start 169.388 99.568) (end 167.64 97.82) (width 0.8) (layer B.Cu) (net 17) (status 30))
 (segment (start 176.276 108.712) (end 176.276 99.568) (width 0.8) (layer B.Cu) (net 17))
 (segment (start 176.276 99.568) (end 169.388 99.568) (width 0.8) (layer B.Cu) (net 17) (status 20))
 (segment (start 176.784 109.22) (end 176.276 108.712) (width 0.8) (layer B.Cu) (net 17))
 (segment (start 176.403 83.185) (end 180.475 83.185) (width 0.8) (layer F.Cu) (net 17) (status 20))
 (segment (start 171.196 88.392) (end 176.403 83.185) (width 0.8) (layer F.Cu) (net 17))
 (segment (start 170.068 88.392) (end 171.196 88.392) (width 0.8) (layer F.Cu) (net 17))
 (segment (start 167.64 90.82) (end 170.068 88.392) (width 0.8) (layer F.Cu) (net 17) (status 10))
 (segment (start 207.895 102.87) (end 218.825 102.87) (width 0.6) (layer F.Cu) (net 19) (status 30))
 (segment (start 213.995 114.735) (end 213.995 116.59) (width 0.6) (layer F.Cu) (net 18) (status 20))
 (segment (start 213.995 109.3) (end 213.995 114.735) (width 0.6) (layer F.Cu) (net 18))
 (segment (start 211.205 106.51) (end 213.995 109.3) (width 0.6) (layer F.Cu) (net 18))
 (segment (start 211.205 105.41) (end 211.205 106.51) (width 0.6) (layer F.Cu) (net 18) (status 10))
 (segment (start 188.595 116.59) (end 188.595 86.615011) (width 0.6) (layer F.Cu) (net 10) (status 10))
 (segment (start 170.639999 79.199999) (end 167.64 76.2) (width 0.6) (layer F.Cu) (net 10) (status 20))
 (segment (start 172.340011 80.900011) (end 170.639999 79.199999) (width 0.6) (layer F.Cu) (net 10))
 (segment (start 182.88 80.900011) (end 172.340011 80.900011) (width 0.6) (layer F.Cu) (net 10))
 (segment (start 188.595 86.615011) (end 182.88 80.900011) (width 0.6) (layer F.Cu) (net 10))
 (segment (start 227.640001 79.199999) (end 230.64 76.2) (width 0.6) (layer F.Cu) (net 3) (status 20))
 (segment (start 224.855001 81.984999) (end 227.640001 79.199999) (width 0.6) (layer F.Cu) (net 3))
 (segment (start 205.105 108.03) (end 205.105 85.09) (width 0.6) (layer F.Cu) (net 3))
 (segment (start 208.210001 81.984999) (end 224.855001 81.984999) (width 0.6) (layer F.Cu) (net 3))
 (segment (start 205.105 85.09) (end 208.210001 81.984999) (width 0.6) (layer F.Cu) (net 3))
 (segment (start 210.355 113.28) (end 205.105 108.03) (width 0.6) (layer F.Cu) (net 3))
 (segment (start 211.455 113.28) (end 210.355 113.28) (width 0.6) (layer F.Cu) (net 3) (status 10))
 (segment (start 213.640001 79.199999) (end 216.64 76.2) (width 0.6) (layer F.Cu) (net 1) (status 20))
 (segment (start 212.939999 79.900001) (end 213.640001 79.199999) (width 0.6) (layer F.Cu) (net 1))
 (segment (start 203.739978 109.493436) (end 202.565 108.318458) (width 0.6) (layer F.Cu) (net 1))
 (segment (start 207.466541 79.900001) (end 212.939999 79.900001) (width 0.6) (layer F.Cu) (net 1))
 (segment (start 206.669998 116.59) (end 203.739978 113.65998) (width 0.6) (layer F.Cu) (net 1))
 (segment (start 202.565 84.801542) (end 207.466541 79.900001) (width 0.6) (layer F.Cu) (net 1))
 (segment (start 208.915 116.59) (end 206.669998 116.59) (width 0.6) (layer F.Cu) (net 1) (status 10))
 (segment (start 202.565 108.318458) (end 202.565 84.801542) (width 0.6) (layer F.Cu) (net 1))
 (segment (start 203.739978 113.65998) (end 203.739978 109.493436) (width 0.6) (layer F.Cu) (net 1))
 (segment (start 220.640001 79.199999) (end 223.64 76.2) (width 0.6) (layer F.Cu) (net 2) (status 20))
 (segment (start 218.939988 80.900012) (end 220.640001 79.199999) (width 0.6) (layer F.Cu) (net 2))
 (segment (start 206.375 113.28) (end 206.375 110.714229) (width 0.6) (layer F.Cu) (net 2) (status 10))
 (segment (start 203.835 108.174229) (end 203.835 84.945771) (width 0.6) (layer F.Cu) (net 2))
 (segment (start 206.375 110.714229) (end 203.835 108.174229) (width 0.6) (layer F.Cu) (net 2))
 (segment (start 207.880759 80.900012) (end 218.939988 80.900012) (width 0.6) (layer F.Cu) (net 2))
 (segment (start 203.835 84.945771) (end 207.880759 80.900012) (width 0.6) (layer F.Cu) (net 2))
 (segment (start 207.06 133.35) (end 206.375 134.035) (width 0.6) (layer F.Cu) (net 11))
 (segment (start 206.375 134.035) (end 206.375 135.89) (width 0.6) (layer F.Cu) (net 11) (status 20))
 (segment (start 224.41 133.35) (end 207.06 133.35) (width 0.6) (layer F.Cu) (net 11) (status 10))
 (segment (start 188.595 147.275) (end 188.64 147.32) (width 0.6) (layer F.Cu) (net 28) (status 30))
 (segment (start 188.595 139.2) (end 188.595 147.275) (width 0.6) (layer F.Cu) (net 28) (status 30))
 (segment (start 183.515 145.445) (end 181.64 147.32) (width 0.6) (layer F.Cu) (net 29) (status 30))
 (segment (start 183.515 139.2) (end 183.515 145.445) (width 0.6) (layer F.Cu) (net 29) (status 30))
 (segment (start 229.614348 147.32) (end 230.64 147.32) (width 0.6) (layer F.Cu) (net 24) (status 30))
 (segment (start 223.449349 141.155001) (end 229.614348 147.32) (width 0.6) (layer F.Cu) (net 24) (status 20))
 (segment (start 212.934999 141.155001) (end 223.449349 141.155001) (width 0.6) (layer F.Cu) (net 24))
 (segment (start 216.535 135.89) (end 214.289998 135.89) (width 0.6) (layer F.Cu) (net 24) (status 10))
 (segment (start 212.794999 141.015001) (end 212.934999 141.155001) (width 0.6) (layer F.Cu) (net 24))
 (segment (start 212.794999 137.384999) (end 212.794999 141.015001) (width 0.6) (layer F.Cu) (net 24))
 (segment (start 214.289998 135.89) (end 212.794999 137.384999) (width 0.6) (layer F.Cu) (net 24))
 (segment (start 220.640001 144.320001) (end 223.64 147.32) (width 0.6) (layer F.Cu) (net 23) (status 20))
 (segment (start 219.195 142.875) (end 220.640001 144.320001) (width 0.6) (layer F.Cu) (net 23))
 (segment (start 212.725 142.875) (end 219.195 142.875) (width 0.6) (layer F.Cu) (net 23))
 (segment (start 211.455 141.605) (end 212.725 142.875) (width 0.6) (layer F.Cu) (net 23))
 (segment (start 201.295 139.675002) (end 203.224998 141.605) (width 0.6) (layer F.Cu) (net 23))
 (segment (start 203.224998 141.605) (end 211.455 141.605) (width 0.6) (layer F.Cu) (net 23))
 (segment (start 201.295 135.89) (end 201.295 139.675002) (width 0.6) (layer F.Cu) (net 23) (status 10))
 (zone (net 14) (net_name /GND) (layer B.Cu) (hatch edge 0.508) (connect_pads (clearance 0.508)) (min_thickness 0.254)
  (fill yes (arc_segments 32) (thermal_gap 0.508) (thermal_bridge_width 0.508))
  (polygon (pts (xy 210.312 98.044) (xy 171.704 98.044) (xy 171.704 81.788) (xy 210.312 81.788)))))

